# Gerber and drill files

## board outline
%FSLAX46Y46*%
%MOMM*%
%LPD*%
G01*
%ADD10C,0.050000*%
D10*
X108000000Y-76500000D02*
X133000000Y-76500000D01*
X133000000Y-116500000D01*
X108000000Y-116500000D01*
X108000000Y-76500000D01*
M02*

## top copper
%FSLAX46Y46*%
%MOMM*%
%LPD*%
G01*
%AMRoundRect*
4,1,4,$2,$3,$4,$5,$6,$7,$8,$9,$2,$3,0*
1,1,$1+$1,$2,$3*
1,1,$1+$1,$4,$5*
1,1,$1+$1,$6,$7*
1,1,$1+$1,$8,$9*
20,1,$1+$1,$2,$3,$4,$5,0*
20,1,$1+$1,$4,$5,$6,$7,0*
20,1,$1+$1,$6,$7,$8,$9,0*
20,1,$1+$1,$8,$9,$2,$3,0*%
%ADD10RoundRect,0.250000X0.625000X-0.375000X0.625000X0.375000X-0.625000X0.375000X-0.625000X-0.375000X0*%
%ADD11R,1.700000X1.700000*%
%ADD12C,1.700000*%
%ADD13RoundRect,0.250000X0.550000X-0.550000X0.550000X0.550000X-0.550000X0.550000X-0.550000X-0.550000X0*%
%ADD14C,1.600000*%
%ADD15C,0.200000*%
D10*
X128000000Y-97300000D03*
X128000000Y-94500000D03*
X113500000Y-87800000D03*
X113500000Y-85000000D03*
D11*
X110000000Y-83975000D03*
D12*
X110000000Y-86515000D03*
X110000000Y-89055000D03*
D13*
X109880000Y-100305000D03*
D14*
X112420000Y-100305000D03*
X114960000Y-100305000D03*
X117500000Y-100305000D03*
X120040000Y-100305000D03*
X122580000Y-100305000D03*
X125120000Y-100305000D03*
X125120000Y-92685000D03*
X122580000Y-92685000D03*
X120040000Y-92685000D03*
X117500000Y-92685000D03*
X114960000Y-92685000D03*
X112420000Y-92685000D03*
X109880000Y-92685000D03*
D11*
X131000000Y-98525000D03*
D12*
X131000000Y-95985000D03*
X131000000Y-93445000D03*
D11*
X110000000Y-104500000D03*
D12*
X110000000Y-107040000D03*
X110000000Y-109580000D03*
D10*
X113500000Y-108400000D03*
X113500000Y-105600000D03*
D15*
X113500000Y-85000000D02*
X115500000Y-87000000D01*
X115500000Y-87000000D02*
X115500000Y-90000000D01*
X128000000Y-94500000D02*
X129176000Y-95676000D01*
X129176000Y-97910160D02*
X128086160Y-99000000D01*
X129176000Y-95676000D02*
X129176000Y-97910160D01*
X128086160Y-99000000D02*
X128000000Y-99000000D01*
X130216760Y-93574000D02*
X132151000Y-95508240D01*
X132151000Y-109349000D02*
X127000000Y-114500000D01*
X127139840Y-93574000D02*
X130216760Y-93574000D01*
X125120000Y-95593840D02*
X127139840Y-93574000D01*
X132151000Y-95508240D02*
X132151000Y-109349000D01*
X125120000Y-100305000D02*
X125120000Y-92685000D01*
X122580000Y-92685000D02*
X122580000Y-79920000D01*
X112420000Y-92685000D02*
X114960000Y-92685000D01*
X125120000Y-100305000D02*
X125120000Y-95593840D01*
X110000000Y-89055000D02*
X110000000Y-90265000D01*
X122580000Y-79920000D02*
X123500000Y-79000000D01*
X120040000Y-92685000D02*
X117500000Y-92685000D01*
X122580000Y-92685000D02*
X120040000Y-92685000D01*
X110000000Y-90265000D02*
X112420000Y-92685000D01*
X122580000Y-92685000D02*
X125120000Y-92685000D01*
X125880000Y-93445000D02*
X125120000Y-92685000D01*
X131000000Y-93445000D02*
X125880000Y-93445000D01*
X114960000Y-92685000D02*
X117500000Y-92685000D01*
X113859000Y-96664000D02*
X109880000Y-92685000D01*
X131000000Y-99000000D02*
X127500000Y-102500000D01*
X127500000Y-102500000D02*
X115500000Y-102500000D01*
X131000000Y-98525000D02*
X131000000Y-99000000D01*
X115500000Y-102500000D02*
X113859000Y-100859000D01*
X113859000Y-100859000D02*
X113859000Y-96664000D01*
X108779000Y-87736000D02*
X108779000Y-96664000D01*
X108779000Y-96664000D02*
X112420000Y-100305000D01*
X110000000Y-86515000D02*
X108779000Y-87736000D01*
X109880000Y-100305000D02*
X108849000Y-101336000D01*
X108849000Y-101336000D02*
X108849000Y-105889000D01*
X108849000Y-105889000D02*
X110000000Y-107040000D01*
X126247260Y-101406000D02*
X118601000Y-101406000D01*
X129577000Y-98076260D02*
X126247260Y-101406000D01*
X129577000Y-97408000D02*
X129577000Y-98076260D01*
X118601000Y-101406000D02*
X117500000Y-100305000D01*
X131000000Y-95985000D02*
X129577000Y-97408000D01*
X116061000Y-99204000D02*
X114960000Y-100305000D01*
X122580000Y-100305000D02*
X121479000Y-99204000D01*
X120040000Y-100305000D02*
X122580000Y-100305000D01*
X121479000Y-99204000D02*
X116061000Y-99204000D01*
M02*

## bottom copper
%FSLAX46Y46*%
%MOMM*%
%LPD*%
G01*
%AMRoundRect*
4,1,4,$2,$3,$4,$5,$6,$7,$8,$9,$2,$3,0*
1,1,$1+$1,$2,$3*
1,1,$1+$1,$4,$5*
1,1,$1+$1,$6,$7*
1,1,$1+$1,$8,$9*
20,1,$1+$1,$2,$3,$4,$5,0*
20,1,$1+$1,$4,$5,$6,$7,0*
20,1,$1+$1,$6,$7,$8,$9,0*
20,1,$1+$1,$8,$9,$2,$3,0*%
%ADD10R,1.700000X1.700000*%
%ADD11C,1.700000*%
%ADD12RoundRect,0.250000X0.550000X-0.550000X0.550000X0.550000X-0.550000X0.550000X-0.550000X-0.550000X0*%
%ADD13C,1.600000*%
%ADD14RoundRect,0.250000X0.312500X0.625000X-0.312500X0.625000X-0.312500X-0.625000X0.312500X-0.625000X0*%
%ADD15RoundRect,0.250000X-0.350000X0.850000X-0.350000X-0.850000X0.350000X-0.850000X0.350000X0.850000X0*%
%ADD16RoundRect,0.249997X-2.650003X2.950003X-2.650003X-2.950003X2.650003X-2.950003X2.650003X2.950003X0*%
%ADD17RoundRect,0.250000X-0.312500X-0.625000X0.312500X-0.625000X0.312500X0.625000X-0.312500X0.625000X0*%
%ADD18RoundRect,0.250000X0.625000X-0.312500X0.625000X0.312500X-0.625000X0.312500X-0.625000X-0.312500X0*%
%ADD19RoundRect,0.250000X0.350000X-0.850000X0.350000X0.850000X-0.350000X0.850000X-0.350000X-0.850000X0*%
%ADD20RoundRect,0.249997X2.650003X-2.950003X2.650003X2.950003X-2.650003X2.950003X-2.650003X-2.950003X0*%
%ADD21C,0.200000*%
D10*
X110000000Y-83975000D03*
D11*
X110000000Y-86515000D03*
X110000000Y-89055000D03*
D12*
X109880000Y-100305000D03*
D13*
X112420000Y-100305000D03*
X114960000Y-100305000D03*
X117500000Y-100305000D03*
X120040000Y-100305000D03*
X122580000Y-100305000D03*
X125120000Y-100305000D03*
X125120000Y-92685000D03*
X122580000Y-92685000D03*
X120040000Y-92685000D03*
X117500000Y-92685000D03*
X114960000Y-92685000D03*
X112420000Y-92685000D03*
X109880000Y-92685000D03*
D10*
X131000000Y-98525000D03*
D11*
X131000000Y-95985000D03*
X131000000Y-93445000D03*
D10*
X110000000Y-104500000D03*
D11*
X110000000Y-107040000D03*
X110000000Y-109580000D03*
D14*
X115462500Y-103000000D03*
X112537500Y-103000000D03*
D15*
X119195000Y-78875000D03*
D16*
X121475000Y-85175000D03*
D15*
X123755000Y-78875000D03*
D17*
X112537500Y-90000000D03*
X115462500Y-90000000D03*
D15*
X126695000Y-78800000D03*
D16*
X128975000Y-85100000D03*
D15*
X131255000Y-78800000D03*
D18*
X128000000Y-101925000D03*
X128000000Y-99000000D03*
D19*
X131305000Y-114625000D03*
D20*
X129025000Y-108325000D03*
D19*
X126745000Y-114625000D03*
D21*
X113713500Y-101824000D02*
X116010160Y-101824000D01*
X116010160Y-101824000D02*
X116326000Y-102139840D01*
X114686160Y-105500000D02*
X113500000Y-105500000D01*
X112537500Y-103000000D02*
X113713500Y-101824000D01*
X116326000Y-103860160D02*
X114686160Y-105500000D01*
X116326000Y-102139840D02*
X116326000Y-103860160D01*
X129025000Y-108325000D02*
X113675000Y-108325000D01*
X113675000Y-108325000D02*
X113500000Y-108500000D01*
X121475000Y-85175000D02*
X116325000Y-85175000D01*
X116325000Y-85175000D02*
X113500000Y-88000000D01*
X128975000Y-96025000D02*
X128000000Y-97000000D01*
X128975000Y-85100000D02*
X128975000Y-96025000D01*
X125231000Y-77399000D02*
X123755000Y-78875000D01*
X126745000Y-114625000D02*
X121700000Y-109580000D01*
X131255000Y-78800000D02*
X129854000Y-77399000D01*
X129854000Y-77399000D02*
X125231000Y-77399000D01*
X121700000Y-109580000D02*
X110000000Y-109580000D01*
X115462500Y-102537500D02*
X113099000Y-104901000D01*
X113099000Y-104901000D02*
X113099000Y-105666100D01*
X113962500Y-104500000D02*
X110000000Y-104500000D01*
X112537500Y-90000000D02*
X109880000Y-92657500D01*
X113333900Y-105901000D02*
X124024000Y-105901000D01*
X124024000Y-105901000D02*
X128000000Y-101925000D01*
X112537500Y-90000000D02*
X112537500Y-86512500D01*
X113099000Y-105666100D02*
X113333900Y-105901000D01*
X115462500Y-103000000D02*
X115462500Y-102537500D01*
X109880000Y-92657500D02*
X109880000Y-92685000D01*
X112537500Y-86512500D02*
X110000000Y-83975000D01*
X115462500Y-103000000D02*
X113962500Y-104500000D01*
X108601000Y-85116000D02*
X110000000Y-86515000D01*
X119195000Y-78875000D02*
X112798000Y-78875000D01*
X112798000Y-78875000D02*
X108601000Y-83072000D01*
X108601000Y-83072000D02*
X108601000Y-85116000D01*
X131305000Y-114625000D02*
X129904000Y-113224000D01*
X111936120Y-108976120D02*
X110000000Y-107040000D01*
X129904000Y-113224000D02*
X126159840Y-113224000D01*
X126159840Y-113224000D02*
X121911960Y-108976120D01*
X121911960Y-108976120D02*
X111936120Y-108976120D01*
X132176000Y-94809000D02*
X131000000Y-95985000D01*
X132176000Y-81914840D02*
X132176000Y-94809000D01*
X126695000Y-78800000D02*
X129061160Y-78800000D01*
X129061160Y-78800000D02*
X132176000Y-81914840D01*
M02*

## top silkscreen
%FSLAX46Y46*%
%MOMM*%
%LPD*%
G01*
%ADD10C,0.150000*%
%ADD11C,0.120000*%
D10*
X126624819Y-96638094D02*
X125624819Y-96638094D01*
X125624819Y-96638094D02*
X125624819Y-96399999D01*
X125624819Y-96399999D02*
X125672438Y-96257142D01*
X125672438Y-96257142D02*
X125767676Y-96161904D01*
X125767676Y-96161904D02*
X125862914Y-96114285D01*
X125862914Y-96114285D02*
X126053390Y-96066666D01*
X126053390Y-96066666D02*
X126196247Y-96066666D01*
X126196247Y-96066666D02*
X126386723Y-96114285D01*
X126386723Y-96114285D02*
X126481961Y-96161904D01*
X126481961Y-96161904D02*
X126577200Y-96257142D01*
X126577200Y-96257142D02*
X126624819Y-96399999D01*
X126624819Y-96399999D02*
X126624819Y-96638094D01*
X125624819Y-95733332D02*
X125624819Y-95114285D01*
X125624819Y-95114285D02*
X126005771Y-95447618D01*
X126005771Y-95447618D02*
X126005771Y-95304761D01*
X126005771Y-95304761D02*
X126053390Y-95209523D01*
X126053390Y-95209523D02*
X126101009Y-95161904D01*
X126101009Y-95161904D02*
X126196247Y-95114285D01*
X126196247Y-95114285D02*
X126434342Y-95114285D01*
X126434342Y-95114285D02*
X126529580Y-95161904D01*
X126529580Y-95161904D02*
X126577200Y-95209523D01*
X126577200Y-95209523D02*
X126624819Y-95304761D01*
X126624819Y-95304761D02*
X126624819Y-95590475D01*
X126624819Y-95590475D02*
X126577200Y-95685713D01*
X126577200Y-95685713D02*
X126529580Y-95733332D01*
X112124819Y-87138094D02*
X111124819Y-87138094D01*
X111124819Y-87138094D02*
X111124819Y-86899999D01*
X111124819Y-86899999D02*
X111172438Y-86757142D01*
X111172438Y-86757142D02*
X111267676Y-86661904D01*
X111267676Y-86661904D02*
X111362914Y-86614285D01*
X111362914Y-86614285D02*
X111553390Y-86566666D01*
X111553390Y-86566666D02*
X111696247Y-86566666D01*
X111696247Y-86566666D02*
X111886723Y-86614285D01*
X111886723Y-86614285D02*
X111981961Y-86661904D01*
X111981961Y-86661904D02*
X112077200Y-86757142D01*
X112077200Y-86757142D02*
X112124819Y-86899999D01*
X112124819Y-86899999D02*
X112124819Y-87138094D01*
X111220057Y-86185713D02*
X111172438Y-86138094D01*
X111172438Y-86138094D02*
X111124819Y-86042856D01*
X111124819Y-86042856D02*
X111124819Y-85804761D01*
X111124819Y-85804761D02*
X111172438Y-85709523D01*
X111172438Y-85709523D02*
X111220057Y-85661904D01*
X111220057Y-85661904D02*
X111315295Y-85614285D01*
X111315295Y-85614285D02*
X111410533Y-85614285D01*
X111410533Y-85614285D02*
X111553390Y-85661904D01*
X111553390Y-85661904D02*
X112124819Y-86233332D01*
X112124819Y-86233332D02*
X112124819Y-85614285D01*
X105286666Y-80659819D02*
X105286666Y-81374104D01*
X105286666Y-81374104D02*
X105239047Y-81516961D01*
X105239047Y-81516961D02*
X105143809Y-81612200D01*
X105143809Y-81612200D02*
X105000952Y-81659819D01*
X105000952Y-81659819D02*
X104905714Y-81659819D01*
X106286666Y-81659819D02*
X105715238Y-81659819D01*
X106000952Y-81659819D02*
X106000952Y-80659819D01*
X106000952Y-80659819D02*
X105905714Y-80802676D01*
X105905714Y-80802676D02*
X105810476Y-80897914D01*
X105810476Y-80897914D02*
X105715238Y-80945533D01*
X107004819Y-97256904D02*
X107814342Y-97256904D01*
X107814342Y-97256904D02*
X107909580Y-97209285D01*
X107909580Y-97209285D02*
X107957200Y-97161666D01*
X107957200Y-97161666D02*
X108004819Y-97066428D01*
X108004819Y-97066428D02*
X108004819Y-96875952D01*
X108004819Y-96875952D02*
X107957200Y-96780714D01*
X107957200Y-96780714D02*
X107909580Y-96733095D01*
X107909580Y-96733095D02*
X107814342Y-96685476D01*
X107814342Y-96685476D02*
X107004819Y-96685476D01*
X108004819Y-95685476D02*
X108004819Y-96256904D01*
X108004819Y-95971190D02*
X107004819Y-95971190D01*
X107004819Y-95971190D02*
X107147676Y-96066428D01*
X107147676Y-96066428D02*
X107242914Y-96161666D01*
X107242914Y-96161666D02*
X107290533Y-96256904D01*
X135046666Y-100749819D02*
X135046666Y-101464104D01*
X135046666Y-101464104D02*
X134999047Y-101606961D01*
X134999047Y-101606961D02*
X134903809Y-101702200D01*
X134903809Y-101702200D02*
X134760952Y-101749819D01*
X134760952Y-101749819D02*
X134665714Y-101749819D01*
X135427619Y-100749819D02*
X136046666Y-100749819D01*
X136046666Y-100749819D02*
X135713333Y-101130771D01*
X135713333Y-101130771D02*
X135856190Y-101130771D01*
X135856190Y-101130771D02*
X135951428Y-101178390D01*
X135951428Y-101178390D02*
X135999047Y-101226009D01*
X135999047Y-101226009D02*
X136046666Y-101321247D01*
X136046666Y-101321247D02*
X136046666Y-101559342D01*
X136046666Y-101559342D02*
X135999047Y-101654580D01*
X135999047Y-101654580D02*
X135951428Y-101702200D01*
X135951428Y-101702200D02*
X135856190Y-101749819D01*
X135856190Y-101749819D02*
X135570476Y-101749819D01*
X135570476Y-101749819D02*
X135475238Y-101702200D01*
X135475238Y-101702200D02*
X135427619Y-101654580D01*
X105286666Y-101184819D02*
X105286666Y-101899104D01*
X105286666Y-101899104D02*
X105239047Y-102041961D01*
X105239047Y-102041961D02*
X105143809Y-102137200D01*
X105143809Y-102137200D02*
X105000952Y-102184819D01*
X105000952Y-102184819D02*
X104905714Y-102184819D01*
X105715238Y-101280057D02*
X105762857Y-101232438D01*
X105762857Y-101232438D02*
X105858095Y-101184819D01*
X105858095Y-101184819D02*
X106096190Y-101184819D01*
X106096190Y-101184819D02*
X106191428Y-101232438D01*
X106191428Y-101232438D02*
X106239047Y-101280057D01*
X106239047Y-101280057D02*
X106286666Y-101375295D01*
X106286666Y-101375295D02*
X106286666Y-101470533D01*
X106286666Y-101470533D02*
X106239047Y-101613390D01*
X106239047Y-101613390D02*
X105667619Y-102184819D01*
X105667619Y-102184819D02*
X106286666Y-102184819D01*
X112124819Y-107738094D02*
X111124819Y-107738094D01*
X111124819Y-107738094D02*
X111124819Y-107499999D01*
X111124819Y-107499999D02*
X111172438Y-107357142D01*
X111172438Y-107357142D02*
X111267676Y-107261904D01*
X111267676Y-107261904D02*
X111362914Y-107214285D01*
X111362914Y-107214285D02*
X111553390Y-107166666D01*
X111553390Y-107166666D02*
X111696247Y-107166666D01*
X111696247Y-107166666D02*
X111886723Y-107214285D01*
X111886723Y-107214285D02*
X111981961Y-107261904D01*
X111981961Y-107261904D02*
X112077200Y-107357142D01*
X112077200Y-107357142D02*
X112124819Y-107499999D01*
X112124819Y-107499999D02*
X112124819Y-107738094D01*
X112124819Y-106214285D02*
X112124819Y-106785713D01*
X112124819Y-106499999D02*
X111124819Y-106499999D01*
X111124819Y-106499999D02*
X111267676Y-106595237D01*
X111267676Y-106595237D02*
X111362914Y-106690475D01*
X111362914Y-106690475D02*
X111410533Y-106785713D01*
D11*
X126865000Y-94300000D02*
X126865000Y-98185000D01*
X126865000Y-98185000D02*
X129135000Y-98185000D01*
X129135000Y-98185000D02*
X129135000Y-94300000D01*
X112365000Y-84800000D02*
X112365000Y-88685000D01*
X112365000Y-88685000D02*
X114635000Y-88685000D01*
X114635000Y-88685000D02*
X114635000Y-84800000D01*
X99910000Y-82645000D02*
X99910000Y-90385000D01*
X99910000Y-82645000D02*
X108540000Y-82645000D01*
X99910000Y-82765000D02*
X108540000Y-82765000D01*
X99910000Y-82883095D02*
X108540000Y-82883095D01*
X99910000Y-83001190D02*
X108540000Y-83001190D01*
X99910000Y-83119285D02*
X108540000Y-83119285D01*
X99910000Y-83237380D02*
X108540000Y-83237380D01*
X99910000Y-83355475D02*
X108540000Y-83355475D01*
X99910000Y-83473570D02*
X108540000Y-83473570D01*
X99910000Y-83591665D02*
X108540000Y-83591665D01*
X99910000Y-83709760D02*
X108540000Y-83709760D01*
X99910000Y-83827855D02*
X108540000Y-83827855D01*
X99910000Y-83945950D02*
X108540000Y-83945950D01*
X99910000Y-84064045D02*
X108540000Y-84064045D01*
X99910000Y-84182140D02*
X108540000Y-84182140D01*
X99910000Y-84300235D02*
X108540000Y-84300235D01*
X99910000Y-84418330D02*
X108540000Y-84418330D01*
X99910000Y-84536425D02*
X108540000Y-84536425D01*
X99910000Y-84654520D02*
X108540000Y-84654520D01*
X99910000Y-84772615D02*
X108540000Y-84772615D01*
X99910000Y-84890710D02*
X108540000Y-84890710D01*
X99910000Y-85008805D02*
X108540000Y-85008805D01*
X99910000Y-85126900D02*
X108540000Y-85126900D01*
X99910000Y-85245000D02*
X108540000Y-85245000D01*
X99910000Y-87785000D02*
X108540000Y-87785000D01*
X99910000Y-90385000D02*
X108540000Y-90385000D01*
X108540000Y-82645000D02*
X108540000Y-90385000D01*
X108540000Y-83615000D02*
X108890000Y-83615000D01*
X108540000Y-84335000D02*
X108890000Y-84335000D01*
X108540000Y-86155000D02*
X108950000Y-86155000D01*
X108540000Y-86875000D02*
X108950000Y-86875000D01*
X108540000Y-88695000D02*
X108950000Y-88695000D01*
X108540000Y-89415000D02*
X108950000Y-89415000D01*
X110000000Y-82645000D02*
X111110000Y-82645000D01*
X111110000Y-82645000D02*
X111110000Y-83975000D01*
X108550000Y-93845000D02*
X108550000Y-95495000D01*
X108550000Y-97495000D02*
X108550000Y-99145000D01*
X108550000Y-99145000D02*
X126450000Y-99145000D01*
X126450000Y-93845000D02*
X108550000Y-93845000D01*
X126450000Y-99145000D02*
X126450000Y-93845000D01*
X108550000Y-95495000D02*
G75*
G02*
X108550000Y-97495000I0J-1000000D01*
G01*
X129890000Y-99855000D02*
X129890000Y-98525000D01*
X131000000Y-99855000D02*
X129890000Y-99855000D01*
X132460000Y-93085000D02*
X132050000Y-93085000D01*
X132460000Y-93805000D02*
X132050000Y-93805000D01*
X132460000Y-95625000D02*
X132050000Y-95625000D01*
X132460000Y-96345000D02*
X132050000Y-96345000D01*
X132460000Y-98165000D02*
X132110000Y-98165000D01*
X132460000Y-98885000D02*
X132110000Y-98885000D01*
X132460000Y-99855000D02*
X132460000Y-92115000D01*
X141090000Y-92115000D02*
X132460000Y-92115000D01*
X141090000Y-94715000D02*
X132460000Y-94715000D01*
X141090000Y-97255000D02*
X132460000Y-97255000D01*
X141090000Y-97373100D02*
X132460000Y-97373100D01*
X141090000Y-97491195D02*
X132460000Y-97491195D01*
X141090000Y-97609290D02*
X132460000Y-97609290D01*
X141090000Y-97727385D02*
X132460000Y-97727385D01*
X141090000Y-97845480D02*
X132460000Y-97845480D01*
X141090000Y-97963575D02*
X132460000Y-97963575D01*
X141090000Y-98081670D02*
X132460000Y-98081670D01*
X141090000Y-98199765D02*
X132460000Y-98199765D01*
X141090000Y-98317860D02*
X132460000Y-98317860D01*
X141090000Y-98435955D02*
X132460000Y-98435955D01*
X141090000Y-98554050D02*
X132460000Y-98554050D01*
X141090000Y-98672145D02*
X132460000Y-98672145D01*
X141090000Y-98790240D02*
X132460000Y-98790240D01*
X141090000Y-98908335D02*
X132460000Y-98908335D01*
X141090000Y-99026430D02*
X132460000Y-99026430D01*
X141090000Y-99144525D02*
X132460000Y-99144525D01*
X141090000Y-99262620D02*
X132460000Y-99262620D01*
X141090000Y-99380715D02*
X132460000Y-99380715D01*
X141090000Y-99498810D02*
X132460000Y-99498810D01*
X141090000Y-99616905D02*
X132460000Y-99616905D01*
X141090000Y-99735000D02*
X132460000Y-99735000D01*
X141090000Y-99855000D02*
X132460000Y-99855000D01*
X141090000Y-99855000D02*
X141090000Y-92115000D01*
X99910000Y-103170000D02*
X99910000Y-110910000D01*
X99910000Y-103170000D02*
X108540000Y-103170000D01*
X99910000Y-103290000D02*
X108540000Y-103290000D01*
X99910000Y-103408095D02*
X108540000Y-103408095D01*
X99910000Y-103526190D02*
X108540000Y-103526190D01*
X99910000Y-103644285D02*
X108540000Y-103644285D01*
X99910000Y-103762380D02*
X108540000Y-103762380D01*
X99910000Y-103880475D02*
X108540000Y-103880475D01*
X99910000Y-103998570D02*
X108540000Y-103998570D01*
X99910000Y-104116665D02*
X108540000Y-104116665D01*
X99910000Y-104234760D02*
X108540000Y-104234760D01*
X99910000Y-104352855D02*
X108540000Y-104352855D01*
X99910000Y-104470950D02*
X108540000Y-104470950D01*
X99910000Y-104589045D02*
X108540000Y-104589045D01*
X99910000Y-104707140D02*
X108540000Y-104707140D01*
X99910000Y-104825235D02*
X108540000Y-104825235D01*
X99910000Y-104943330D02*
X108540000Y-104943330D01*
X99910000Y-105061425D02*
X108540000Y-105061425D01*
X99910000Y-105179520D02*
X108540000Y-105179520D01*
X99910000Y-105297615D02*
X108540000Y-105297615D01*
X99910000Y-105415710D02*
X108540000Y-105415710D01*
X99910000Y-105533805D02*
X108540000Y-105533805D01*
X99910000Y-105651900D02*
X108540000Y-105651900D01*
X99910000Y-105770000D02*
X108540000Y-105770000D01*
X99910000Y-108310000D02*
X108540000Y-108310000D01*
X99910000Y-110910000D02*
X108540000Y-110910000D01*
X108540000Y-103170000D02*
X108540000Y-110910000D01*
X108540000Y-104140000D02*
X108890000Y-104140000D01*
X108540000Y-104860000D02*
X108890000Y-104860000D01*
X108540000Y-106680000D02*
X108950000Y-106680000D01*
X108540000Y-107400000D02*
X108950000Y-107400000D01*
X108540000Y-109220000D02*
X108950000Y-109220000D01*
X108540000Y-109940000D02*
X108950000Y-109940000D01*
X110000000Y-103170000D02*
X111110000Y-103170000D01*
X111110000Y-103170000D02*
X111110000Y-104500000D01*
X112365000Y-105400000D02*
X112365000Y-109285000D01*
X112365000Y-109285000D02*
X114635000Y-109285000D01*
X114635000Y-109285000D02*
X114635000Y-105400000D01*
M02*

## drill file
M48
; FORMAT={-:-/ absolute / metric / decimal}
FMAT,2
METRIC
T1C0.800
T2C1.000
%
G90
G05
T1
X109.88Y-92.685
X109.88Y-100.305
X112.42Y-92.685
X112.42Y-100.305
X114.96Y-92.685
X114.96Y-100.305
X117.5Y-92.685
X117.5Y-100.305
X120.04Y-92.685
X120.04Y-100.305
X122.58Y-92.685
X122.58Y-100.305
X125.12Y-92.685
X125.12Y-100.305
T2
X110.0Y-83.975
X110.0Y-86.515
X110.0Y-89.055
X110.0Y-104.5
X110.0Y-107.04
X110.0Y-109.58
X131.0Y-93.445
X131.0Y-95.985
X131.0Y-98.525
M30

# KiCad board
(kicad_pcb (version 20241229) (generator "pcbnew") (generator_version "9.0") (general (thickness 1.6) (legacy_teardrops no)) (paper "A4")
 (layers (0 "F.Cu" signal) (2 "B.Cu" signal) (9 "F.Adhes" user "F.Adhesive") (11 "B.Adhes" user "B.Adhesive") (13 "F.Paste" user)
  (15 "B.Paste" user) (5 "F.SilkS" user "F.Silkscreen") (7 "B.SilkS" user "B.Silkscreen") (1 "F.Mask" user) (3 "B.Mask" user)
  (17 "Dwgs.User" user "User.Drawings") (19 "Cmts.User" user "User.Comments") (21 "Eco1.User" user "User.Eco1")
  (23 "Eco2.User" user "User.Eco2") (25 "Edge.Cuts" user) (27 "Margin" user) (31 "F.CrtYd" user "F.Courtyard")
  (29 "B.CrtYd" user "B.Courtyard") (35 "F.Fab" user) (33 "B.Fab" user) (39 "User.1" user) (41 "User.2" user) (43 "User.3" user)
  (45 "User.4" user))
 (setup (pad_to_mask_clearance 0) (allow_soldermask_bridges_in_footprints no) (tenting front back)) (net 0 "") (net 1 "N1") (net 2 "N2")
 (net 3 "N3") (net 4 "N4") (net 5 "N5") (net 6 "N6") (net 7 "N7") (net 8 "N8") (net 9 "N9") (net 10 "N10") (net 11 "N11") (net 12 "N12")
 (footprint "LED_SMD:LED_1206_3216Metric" (layer "F.Cu") (at 128 95.9 90)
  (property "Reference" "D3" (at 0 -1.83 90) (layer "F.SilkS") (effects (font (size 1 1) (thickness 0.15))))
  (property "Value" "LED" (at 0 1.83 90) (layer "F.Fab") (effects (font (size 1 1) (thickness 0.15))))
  (fp_line (start 1.6 -1.135) (end -2.285 -1.135) (stroke (width 0.12) (type solid)) (layer "F.SilkS"))
  (fp_line (start -2.285 -1.135) (end -2.285 1.135) (stroke (width 0.12) (type solid)) (layer "F.SilkS"))
  (fp_line (start -2.285 1.135) (end 1.6 1.135) (stroke (width 0.12) (type solid)) (layer "F.SilkS"))
  (pad "1" smd roundrect (at -1.4 0 90) (size 1.25 1.75) (layers "F.Cu" "F.Mask" "F.Paste") (roundrect_rratio 0.2) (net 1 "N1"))
  (pad "2" smd roundrect (at 1.4 0 90) (size 1.25 1.75) (layers "F.Cu" "F.Mask" "F.Paste") (roundrect_rratio 0.2) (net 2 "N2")))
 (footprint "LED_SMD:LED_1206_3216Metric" (layer "F.Cu") (at 113.5 86.4 90)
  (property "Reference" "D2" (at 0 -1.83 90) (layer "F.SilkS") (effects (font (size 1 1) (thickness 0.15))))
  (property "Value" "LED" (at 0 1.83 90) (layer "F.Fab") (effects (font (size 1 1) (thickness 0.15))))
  (fp_line (start 1.6 -1.135) (end -2.285 -1.135) (stroke (width 0.12) (type solid)) (layer "F.SilkS"))
  (fp_line (start -2.285 -1.135) (end -2.285 1.135) (stroke (width 0.12) (type solid)) (layer "F.SilkS"))
  (fp_line (start -2.285 1.135) (end 1.6 1.135) (stroke (width 0.12) (type solid)) (layer "F.SilkS"))
  (pad "1" smd roundrect (at -1.4 0 90) (size 1.25 1.75) (layers "F.Cu" "F.Mask" "F.Paste") (roundrect_rratio 0.2) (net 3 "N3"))
  (pad "2" smd roundrect (at 1.4 0 90) (size 1.25 1.75) (layers "F.Cu" "F.Mask" "F.Paste") (roundrect_rratio 0.2) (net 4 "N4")))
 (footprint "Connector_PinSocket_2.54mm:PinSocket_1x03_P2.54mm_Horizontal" (layer "F.Cu") (at 110 83.975)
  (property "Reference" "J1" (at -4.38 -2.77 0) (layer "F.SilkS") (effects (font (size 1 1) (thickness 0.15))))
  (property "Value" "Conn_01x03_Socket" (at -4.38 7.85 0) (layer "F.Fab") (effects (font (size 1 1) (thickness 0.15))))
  (fp_line (start -10.09 -1.33) (end -10.09 6.41) (stroke (width 0.12) (type solid)) (layer "F.SilkS"))
  (fp_line (start -10.09 -1.33) (end -1.46 -1.33) (stroke (width 0.12) (type solid)) (layer "F.SilkS"))
  (fp_line (start -10.09 -1.21) (end -1.46 -1.21) (stroke (width 0.12) (type solid)) (layer "F.SilkS"))
  (fp_line (start -10.09 -1.091905) (end -1.46 -1.091905) (stroke (width 0.12) (type solid)) (layer "F.SilkS"))
  (fp_line (start -10.09 -0.97381) (end -1.46 -0.97381) (stroke (width 0.12) (type solid)) (layer "F.SilkS"))
  (fp_line (start -10.09 -0.855715) (end -1.46 -0.855715) (stroke (width 0.12) (type solid)) (layer "F.SilkS"))
  (fp_line (start -10.09 -0.73762) (end -1.46 -0.73762) (stroke (width 0.12) (type solid)) (layer "F.SilkS"))
  (fp_line (start -10.09 -0.619525) (end -1.46 -0.619525) (stroke (width 0.12) (type solid)) (layer "F.SilkS"))
  (fp_line (start -10.09 -0.50143) (end -1.46 -0.50143) (stroke (width 0.12) (type solid)) (layer "F.SilkS"))
  (fp_line (start -10.09 -0.383335) (end -1.46 -0.383335) (stroke (width 0.12) (type solid)) (layer "F.SilkS"))
  (fp_line (start -10.09 -0.26524) (end -1.46 -0.26524) (stroke (width 0.12) (type solid)) (layer "F.SilkS"))
  (fp_line (start -10.09 -0.147145) (end -1.46 -0.147145) (stroke (width 0.12) (type solid)) (layer "F.SilkS"))
  (fp_line (start -10.09 -0.02905) (end -1.46 -0.02905) (stroke (width 0.12) (type solid)) (layer "F.SilkS"))
  (fp_line (start -10.09 0.089045) (end -1.46 0.089045) (stroke (width 0.12) (type solid)) (layer "F.SilkS"))
  (fp_line (start -10.09 0.20714) (end -1.46 0.20714) (stroke (width 0.12) (type solid)) (layer "F.SilkS"))
  (fp_line (start -10.09 0.325235) (end -1.46 0.325235) (stroke (width 0.12) (type solid)) (layer "F.SilkS"))
  (fp_line (start -10.09 0.44333) (end -1.46 0.44333) (stroke (width 0.12) (type solid)) (layer "F.SilkS"))
  (fp_line (start -10.09 0.561425) (end -1.46 0.561425) (stroke (width 0.12) (type solid)) (layer "F.SilkS"))
  (fp_line (start -10.09 0.67952) (end -1.46 0.67952) (stroke (width 0.12) (type solid)) (layer "F.SilkS"))
  (fp_line (start -10.09 0.797615) (end -1.46 0.797615) (stroke (width 0.12) (type solid)) (layer "F.SilkS"))
  (fp_line (start -10.09 0.91571) (end -1.46 0.91571) (stroke (width 0.12) (type solid)) (layer "F.SilkS"))
  (fp_line (start -10.09 1.033805) (end -1.46 1.033805) (stroke (width 0.12) (type solid)) (layer "F.SilkS"))
  (fp_line (start -10.09 1.1519) (end -1.46 1.1519) (stroke (width 0.12) (type solid)) (layer "F.SilkS"))
  (fp_line (start -10.09 1.27) (end -1.46 1.27) (stroke (width 0.12) (type solid)) (layer "F.SilkS"))
  (fp_line (start -10.09 3.81) (end -1.46 3.81) (stroke (width 0.12) (type solid)) (layer "F.SilkS"))
  (fp_line (start -10.09 6.41) (end -1.46 6.41) (stroke (width 0.12) (type solid)) (layer "F.SilkS"))
  (fp_line (start -1.46 -1.33) (end -1.46 6.41) (stroke (width 0.12) (type solid)) (layer "F.SilkS"))
  (fp_line (start -1.46 -0.36) (end -1.11 -0.36) (stroke (width 0.12) (type solid)) (layer "F.SilkS"))
  (fp_line (start -1.46 0.36) (end -1.11 0.36) (stroke (width 0.12) (type solid)) (layer "F.SilkS"))
  (fp_line (start -1.46 2.18) (end -1.05 2.18) (stroke (width 0.12) (type solid)) (layer "F.SilkS"))
  (fp_line (start -1.46 2.9) (end -1.05 2.9) (stroke (width 0.12) (type solid)) (layer "F.SilkS"))
  (fp_line (start -1.46 4.72) (end -1.05 4.72) (stroke (width 0.12) (type solid)) (layer "F.SilkS"))
  (fp_line (start -1.46 5.44) (end -1.05 5.44) (stroke (width 0.12) (type solid)) (layer "F.SilkS"))
  (fp_line (start 0 -1.33) (end 1.11 -1.33) (stroke (width 0.12) (type solid)) (layer "F.SilkS"))
  (fp_line (start 1.11 -1.33) (end 1.11 0) (stroke (width 0.12) (type solid)) (layer "F.SilkS"))
  (pad "1" thru_hole rect (at 0 0) (size 1.7 1.7) (drill 1) (layers "*.Cu" "*.Mask") (remove_unused_layers no) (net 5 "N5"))
  (pad "2" thru_hole circle (at 0 2.54) (size 1.7 1.7) (drill 1) (layers "*.Cu" "*.Mask") (remove_unused_layers no) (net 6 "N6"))
  (pad "3" thru_hole circle (at 0 5.08) (size 1.7 1.7) (drill 1) (layers "*.Cu" "*.Mask") (remove_unused_layers no) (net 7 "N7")))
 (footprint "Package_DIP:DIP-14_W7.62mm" (layer "F.Cu") (at 109.88 100.305 90)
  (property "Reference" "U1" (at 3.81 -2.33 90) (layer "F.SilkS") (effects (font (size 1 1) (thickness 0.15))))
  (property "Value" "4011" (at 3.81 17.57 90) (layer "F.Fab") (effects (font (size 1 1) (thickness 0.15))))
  (fp_line (start 6.46 -1.33) (end 4.81 -1.33) (stroke (width 0.12) (type solid)) (layer "F.SilkS"))
  (fp_line (start 2.81 -1.33) (end 1.16 -1.33) (stroke (width 0.12) (type solid)) (layer "F.SilkS"))
  (fp_line (start 1.16 -1.33) (end 1.16 16.57) (stroke (width 0.12) (type solid)) (layer "F.SilkS"))
  (fp_line (start 6.46 16.57) (end 6.46 -1.33) (stroke (width 0.12) (type solid)) (layer "F.SilkS"))
  (fp_line (start 1.16 16.57) (end 6.46 16.57) (stroke (width 0.12) (type solid)) (layer "F.SilkS"))
  (fp_arc (start 4.81 -1.33) (mid 3.81 -0.33) (end 2.81 -1.33) (stroke (width 0.12) (type solid)) (layer "F.SilkS"))
  (pad "1" thru_hole roundrect (at 0 0 90) (size 1.6 1.6) (drill 0.8) (layers "*.Cu" "*.Mask") (remove_unused_layers no)
   (roundrect_rratio 0.15625) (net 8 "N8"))
  (pad "2" thru_hole circle (at 0 2.54 90) (size 1.6 1.6) (drill 0.8) (layers "*.Cu" "*.Mask") (remove_unused_layers no) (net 6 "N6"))
  (pad "3" thru_hole circle (at 0 5.08 90) (size 1.6 1.6) (drill 0.8) (layers "*.Cu" "*.Mask") (remove_unused_layers no) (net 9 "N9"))
  (pad "4" thru_hole circle (at 0 7.62 90) (size 1.6 1.6) (drill 0.8) (layers "*.Cu" "*.Mask") (remove_unused_layers no) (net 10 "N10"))
  (pad "5" thru_hole circle (at 0 10.16 90) (size 1.6 1.6) (drill 0.8) (layers "*.Cu" "*.Mask") (remove_unused_layers no) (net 9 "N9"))
  (pad "6" thru_hole circle (at 0 12.7 90) (size 1.6 1.6) (drill 0.8) (layers "*.Cu" "*.Mask") (remove_unused_layers no) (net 9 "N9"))
  (pad "7" thru_hole circle (at 0 15.24 90) (size 1.6 1.6) (drill 0.8) (layers "*.Cu" "*.Mask") (remove_unused_layers no) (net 7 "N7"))
  (pad "8" thru_hole circle (at 7.62 15.24 90) (size 1.6 1.6) (drill 0.8) (layers "*.Cu" "*.Mask") (remove_unused_layers no) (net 7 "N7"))
  (pad "9" thru_hole circle (at 7.62 12.7 90) (size 1.6 1.6) (drill 0.8) (layers "*.Cu" "*.Mask") (remove_unused_layers no) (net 7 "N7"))
  (pad "10" thru_hole circle (at 7.62 10.16 90) (size 1.6 1.6) (drill 0.8) (layers "*.Cu" "*.Mask") (remove_unused_layers no) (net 7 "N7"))
  (pad "11" thru_hole circle (at 7.62 7.62 90) (size 1.6 1.6) (drill 0.8) (layers "*.Cu" "*.Mask") (remove_unused_layers no) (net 7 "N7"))
  (pad "12" thru_hole circle (at 7.62 5.08 90) (size 1.6 1.6) (drill 0.8) (layers "*.Cu" "*.Mask") (remove_unused_layers no) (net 7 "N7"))
  (pad "13" thru_hole circle (at 7.62 2.54 90) (size 1.6 1.6) (drill 0.8) (layers "*.Cu" "*.Mask") (remove_unused_layers no) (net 7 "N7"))
  (pad "14" thru_hole circle (at 7.62 0 90) (size 1.6 1.6) (drill 0.8) (layers "*.Cu" "*.Mask") (remove_unused_layers no) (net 5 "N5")))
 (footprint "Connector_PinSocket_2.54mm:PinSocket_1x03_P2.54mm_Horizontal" (layer "F.Cu") (at 131 98.525 180)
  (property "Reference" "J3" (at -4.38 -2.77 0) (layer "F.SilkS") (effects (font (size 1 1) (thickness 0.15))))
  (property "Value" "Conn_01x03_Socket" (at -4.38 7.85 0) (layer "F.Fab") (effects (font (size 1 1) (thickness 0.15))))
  (fp_line (start 1.11 -1.33) (end 1.11 0) (stroke (width 0.12) (type solid)) (layer "F.SilkS"))
  (fp_line (start 0 -1.33) (end 1.11 -1.33) (stroke (width 0.12) (type solid)) (layer "F.SilkS"))
  (fp_line (start -1.46 5.44) (end -1.05 5.44) (stroke (width 0.12) (type solid)) (layer "F.SilkS"))
  (fp_line (start -1.46 4.72) (end -1.05 4.72) (stroke (width 0.12) (type solid)) (layer "F.SilkS"))
  (fp_line (start -1.46 2.9) (end -1.05 2.9) (stroke (width 0.12) (type solid)) (layer "F.SilkS"))
  (fp_line (start -1.46 2.18) (end -1.05 2.18) (stroke (width 0.12) (type solid)) (layer "F.SilkS"))
  (fp_line (start -1.46 0.36) (end -1.11 0.36) (stroke (width 0.12) (type solid)) (layer "F.SilkS"))
  (fp_line (start -1.46 -0.36) (end -1.11 -0.36) (stroke (width 0.12) (type solid)) (layer "F.SilkS"))
  (fp_line (start -1.46 -1.33) (end -1.46 6.41) (stroke (width 0.12) (type solid)) (layer "F.SilkS"))
  (fp_line (start -10.09 6.41) (end -1.46 6.41) (stroke (width 0.12) (type solid)) (layer "F.SilkS"))
  (fp_line (start -10.09 3.81) (end -1.46 3.81) (stroke (width 0.12) (type solid)) (layer "F.SilkS"))
  (fp_line (start -10.09 1.27) (end -1.46 1.27) (stroke (width 0.12) (type solid)) (layer "F.SilkS"))
  (fp_line (start -10.09 1.1519) (end -1.46 1.1519) (stroke (width 0.12) (type solid)) (layer "F.SilkS"))
  (fp_line (start -10.09 1.033805) (end -1.46 1.033805) (stroke (width 0.12) (type solid)) (layer "F.SilkS"))
  (fp_line (start -10.09 0.91571) (end -1.46 0.91571) (stroke (width 0.12) (type solid)) (layer "F.SilkS"))
  (fp_line (start -10.09 0.797615) (end -1.46 0.797615) (stroke (width 0.12) (type solid)) (layer "F.SilkS"))
  (fp_line (start -10.09 0.67952) (end -1.46 0.67952) (stroke (width 0.12) (type solid)) (layer "F.SilkS"))
  (fp_line (start -10.09 0.561425) (end -1.46 0.561425) (stroke (width 0.12) (type solid)) (layer "F.SilkS"))
  (fp_line (start -10.09 0.44333) (end -1.46 0.44333) (stroke (width 0.12) (type solid)) (layer "F.SilkS"))
  (fp_line (start -10.09 0.325235) (end -1.46 0.325235) (stroke (width 0.12) (type solid)) (layer "F.SilkS"))
  (fp_line (start -10.09 0.20714) (end -1.46 0.20714) (stroke (width 0.12) (type solid)) (layer "F.SilkS"))
  (fp_line (start -10.09 0.089045) (end -1.46 0.089045) (stroke (width 0.12) (type solid)) (layer "F.SilkS"))
  (fp_line (start -10.09 -0.02905) (end -1.46 -0.02905) (stroke (width 0.12) (type solid)) (layer "F.SilkS"))
  (fp_line (start -10.09 -0.147145) (end -1.46 -0.147145) (stroke (width 0.12) (type solid)) (layer "F.SilkS"))
  (fp_line (start -10.09 -0.26524) (end -1.46 -0.26524) (stroke (width 0.12) (type solid)) (layer "F.SilkS"))
  (fp_line (start -10.09 -0.383335) (end -1.46 -0.383335) (stroke (width 0.12) (type solid)) (layer "F.SilkS"))
  (fp_line (start -10.09 -0.50143) (end -1.46 -0.50143) (stroke (width 0.12) (type solid)) (layer "F.SilkS"))
  (fp_line (start -10.09 -0.619525) (end -1.46 -0.619525) (stroke (width 0.12) (type solid)) (layer "F.SilkS"))
  (fp_line (start -10.09 -0.73762) (end -1.46 -0.73762) (stroke (width 0.12) (type solid)) (layer "F.SilkS"))
  (fp_line (start -10.09 -0.855715) (end -1.46 -0.855715) (stroke (width 0.12) (type solid)) (layer "F.SilkS"))
  (fp_line (start -10.09 -0.97381) (end -1.46 -0.97381) (stroke (width 0.12) (type solid)) (layer "F.SilkS"))
  (fp_line (start -10.09 -1.091905) (end -1.46 -1.091905) (stroke (width 0.12) (type solid)) (layer "F.SilkS"))
  (fp_line (start -10.09 -1.21) (end -1.46 -1.21) (stroke (width 0.12) (type solid)) (layer "F.SilkS"))
  (fp_line (start -10.09 -1.33) (end -1.46 -1.33) (stroke (width 0.12) (type solid)) (layer "F.SilkS"))
  (fp_line (start -10.09 -1.33) (end -10.09 6.41) (stroke (width 0.12) (type solid)) (layer "F.SilkS"))
  (pad "1" thru_hole rect (at 0 0 180) (size 1.7 1.7) (drill 1) (layers "*.Cu" "*.Mask") (remove_unused_layers no) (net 5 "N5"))
  (pad "2" thru_hole circle (at 0 2.54 180) (size 1.7 1.7) (drill 1) (layers "*.Cu" "*.Mask") (remove_unused_layers no) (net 10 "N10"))
  (pad "3" thru_hole circle (at 0 5.08 180) (size 1.7 1.7) (drill 1) (layers "*.Cu" "*.Mask") (remove_unused_layers no) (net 7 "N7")))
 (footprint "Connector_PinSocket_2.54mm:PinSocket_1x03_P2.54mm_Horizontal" (layer "F.Cu") (at 110 104.5)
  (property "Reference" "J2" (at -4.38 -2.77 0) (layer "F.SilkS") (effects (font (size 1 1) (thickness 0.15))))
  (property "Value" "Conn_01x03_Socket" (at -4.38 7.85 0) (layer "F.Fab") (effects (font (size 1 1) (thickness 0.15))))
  (fp_line (start -10.09 -1.33) (end -10.09 6.41) (stroke (width 0.12) (type solid)) (layer "F.SilkS"))
  (fp_line (start -10.09 -1.33) (end -1.46 -1.33) (stroke (width 0.12) (type solid)) (layer "F.SilkS"))
  (fp_line (start -10.09 -1.21) (end -1.46 -1.21) (stroke (width 0.12) (type solid)) (layer "F.SilkS"))
  (fp_line (start -10.09 -1.091905) (end -1.46 -1.091905) (stroke (width 0.12) (type solid)) (layer "F.SilkS"))
  (fp_line (start -10.09 -0.97381) (end -1.46 -0.97381) (stroke (width 0.12) (type solid)) (layer "F.SilkS"))
  (fp_line (start -10.09 -0.855715) (end -1.46 -0.855715) (stroke (width 0.12) (type solid)) (layer "F.SilkS"))
  (fp_line (start -10.09 -0.73762) (end -1.46 -0.73762) (stroke (width 0.12) (type solid)) (layer "F.SilkS"))
  (fp_line (start -10.09 -0.619525) (end -1.46 -0.619525) (stroke (width 0.12) (type solid)) (layer "F.SilkS"))
  (fp_line (start -10.09 -0.50143) (end -1.46 -0.50143) (stroke (width 0.12) (type solid)) (layer "F.SilkS"))
  (fp_line (start -10.09 -0.383335) (end -1.46 -0.383335) (stroke (width 0.12) (type solid)) (layer "F.SilkS"))
  (fp_line (start -10.09 -0.26524) (end -1.46 -0.26524) (stroke (width 0.12) (type solid)) (layer "F.SilkS"))
  (fp_line (start -10.09 -0.147145) (end -1.46 -0.147145) (stroke (width 0.12) (type solid)) (layer "F.SilkS"))
  (fp_line (start -10.09 -0.02905) (end -1.46 -0.02905) (stroke (width 0.12) (type solid)) (layer "F.SilkS"))
  (fp_line (start -10.09 0.089045) (end -1.46 0.089045) (stroke (width 0.12) (type solid)) (layer "F.SilkS"))
  (fp_line (start -10.09 0.20714) (end -1.46 0.20714) (stroke (width 0.12) (type solid)) (layer "F.SilkS"))
  (fp_line (start -10.09 0.325235) (end -1.46 0.325235) (stroke (width 0.12) (type solid)) (layer "F.SilkS"))
  (fp_line (start -10.09 0.44333) (end -1.46 0.44333) (stroke (width 0.12) (type solid)) (layer "F.SilkS"))
  (fp_line (start -10.09 0.561425) (end -1.46 0.561425) (stroke (width 0.12) (type solid)) (layer "F.SilkS"))
  (fp_line (start -10.09 0.67952) (end -1.46 0.67952) (stroke (width 0.12) (type solid)) (layer "F.SilkS"))
  (fp_line (start -10.09 0.797615) (end -1.46 0.797615) (stroke (width 0.12) (type solid)) (layer "F.SilkS"))
  (fp_line (start -10.09 0.91571) (end -1.46 0.91571) (stroke (width 0.12) (type solid)) (layer "F.SilkS"))
  (fp_line (start -10.09 1.033805) (end -1.46 1.033805) (stroke (width 0.12) (type solid)) (layer "F.SilkS"))
  (fp_line (start -10.09 1.1519) (end -1.46 1.1519) (stroke (width 0.12) (type solid)) (layer "F.SilkS"))
  (fp_line (start -10.09 1.27) (end -1.46 1.27) (stroke (width 0.12) (type solid)) (layer "F.SilkS"))
  (fp_line (start -10.09 3.81) (end -1.46 3.81) (stroke (width 0.12) (type solid)) (layer "F.SilkS"))
  (fp_line (start -10.09 6.41) (end -1.46 6.41) (stroke (width 0.12) (type solid)) (layer "F.SilkS"))
  (fp_line (start -1.46 -1.33) (end -1.46 6.41) (stroke (width 0.12) (type solid)) (layer "F.SilkS"))
  (fp_line (start -1.46 -0.36) (end -1.11 -0.36) (stroke (width 0.12) (type solid)) (layer "F.SilkS"))
  (fp_line (start -1.46 0.36) (end -1.11 0.36) (stroke (width 0.12) (type solid)) (layer "F.SilkS"))
  (fp_line (start -1.46 2.18) (end -1.05 2.18) (stroke (width 0.12) (type solid)) (layer "F.SilkS"))
  (fp_line (start -1.46 2.9) (end -1.05 2.9) (stroke (width 0.12) (type solid)) (layer "F.SilkS"))
  (fp_line (start -1.46 4.72) (end -1.05 4.72) (stroke (width 0.12) (type solid)) (layer "F.SilkS"))
  (fp_line (start -1.46 5.44) (end -1.05 5.44) (stroke (width 0.12) (type solid)) (layer "F.SilkS"))
  (fp_line (start 0 -1.33) (end 1.11 -1.33) (stroke (width 0.12) (type solid)) (layer "F.SilkS"))
  (fp_line (start 1.11 -1.33) (end 1.11 0) (stroke (width 0.12) (type solid)) (layer "F.SilkS"))
  (pad "1" thru_hole rect (at 0 0) (size 1.7 1.7) (drill 1) (layers "*.Cu" "*.Mask") (remove_unused_layers no) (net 5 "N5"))
  (pad "2" thru_hole circle (at 0 2.54) (size 1.7 1.7) (drill 1) (layers "*.Cu" "*.Mask") (remove_unused_layers no) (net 8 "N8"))
  (pad "3" thru_hole circle (at 0 5.08) (size 1.7 1.7) (drill 1) (layers "*.Cu" "*.Mask") (remove_unused_layers no) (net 7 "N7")))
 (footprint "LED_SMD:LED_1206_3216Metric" (layer "F.Cu") (at 113.5 107 90)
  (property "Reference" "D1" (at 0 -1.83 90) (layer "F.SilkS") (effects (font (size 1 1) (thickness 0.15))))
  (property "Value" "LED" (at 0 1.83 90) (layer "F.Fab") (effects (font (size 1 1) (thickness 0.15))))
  (fp_line (start 1.6 -1.135) (end -2.285 -1.135) (stroke (width 0.12) (type solid)) (layer "F.SilkS"))
  (fp_line (start -2.285 -1.135) (end -2.285 1.135) (stroke (width 0.12) (type solid)) (layer "F.SilkS"))
  (fp_line (start -2.285 1.135) (end 1.6 1.135) (stroke (width 0.12) (type solid)) (layer "F.SilkS"))
  (pad "1" smd roundrect (at -1.4 0 90) (size 1.25 1.75) (layers "F.Cu" "F.Mask" "F.Paste") (roundrect_rratio 0.2) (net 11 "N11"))
  (pad "2" smd roundrect (at 1.4 0 90) (size 1.25 1.75) (layers "F.Cu" "F.Mask" "F.Paste") (roundrect_rratio 0.2) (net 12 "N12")))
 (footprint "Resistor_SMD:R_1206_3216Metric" (layer "B.Cu") (at 114 103 180)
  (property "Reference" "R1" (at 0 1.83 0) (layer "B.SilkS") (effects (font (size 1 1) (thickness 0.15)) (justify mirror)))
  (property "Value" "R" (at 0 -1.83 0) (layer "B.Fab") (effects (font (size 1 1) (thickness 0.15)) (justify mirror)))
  (pad "1" smd roundrect (at -1.4625 0 180) (size 1.125 1.75) (layers "B.Cu" "B.Mask" "B.Paste") (roundrect_rratio 0.222222) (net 5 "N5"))
  (pad "2" smd roundrect (at 1.4625 0 180) (size 1.125 1.75) (layers "B.Cu" "B.Mask" "B.Paste") (roundrect_rratio 0.222222) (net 12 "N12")))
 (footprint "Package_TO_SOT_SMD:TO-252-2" (layer "B.Cu") (at 121.475 83.915 -90)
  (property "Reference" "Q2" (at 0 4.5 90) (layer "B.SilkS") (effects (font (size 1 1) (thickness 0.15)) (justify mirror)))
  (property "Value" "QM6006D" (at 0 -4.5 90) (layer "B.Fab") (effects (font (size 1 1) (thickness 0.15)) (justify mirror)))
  (pad "" smd roundrect (at -0.415 -1.525 270) (size 3.05 2.75) (layers "B.Paste") (roundrect_rratio 0.090909))
  (pad "" smd roundrect (at -0.415 1.525 270) (size 3.05 2.75) (layers "B.Paste") (roundrect_rratio 0.090909))
  (pad "" smd roundrect (at 2.935 -1.525 270) (size 3.05 2.75) (layers "B.Paste") (roundrect_rratio 0.090909))
  (pad "" smd roundrect (at 2.935 1.525 270) (size 3.05 2.75) (layers "B.Paste") (roundrect_rratio 0.090909))
  (pad "1" smd roundrect (at -5.04 2.28 270) (size 2.2 1.2) (layers "B.Cu" "B.Mask" "B.Paste") (roundrect_rratio 0.208333) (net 6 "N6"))
  (pad "2" smd roundrect (at 1.26 0 270) (size 6.4 5.8) (layers "B.Cu" "B.Mask") (roundrect_rratio 0.043103) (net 3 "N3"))
  (pad "3" smd roundrect (at -5.04 -2.28 270) (size 2.2 1.2) (layers "B.Cu" "B.Mask" "B.Paste") (roundrect_rratio 0.208333) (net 7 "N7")))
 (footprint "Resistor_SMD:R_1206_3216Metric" (layer "B.Cu") (at 114 90)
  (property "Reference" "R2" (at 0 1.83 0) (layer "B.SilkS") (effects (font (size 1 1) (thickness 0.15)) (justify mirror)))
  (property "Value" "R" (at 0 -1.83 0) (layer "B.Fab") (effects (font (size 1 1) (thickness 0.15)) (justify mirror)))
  (pad "1" smd roundrect (at -1.4625 0) (size 1.125 1.75) (layers "B.Cu" "B.Mask" "B.Paste") (roundrect_rratio 0.222222) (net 5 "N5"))
  (pad "2" smd roundrect (at 1.4625 0) (size 1.125 1.75) (layers "B.Cu" "B.Mask" "B.Paste") (roundrect_rratio 0.222222) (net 4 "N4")))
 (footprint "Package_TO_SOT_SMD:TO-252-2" (layer "B.Cu") (at 128.975 83.84 -90)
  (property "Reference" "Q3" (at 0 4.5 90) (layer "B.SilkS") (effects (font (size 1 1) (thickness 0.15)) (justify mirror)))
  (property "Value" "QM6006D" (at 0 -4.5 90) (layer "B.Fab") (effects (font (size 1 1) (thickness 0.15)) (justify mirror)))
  (pad "" smd roundrect (at -0.415 -1.525 270) (size 3.05 2.75) (layers "B.Paste") (roundrect_rratio 0.090909))
  (pad "" smd roundrect (at -0.415 1.525 270) (size 3.05 2.75) (layers "B.Paste") (roundrect_rratio 0.090909))
  (pad "" smd roundrect (at 2.935 -1.525 270) (size 3.05 2.75) (layers "B.Paste") (roundrect_rratio 0.090909))
  (pad "" smd roundrect (at 2.935 1.525 270) (size 3.05 2.75) (layers "B.Paste") (roundrect_rratio 0.090909))
  (pad "1" smd roundrect (at -5.04 2.28 270) (size 2.2 1.2) (layers "B.Cu" "B.Mask" "B.Paste") (roundrect_rratio 0.208333) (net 10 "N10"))
  (pad "2" smd roundrect (at 1.26 0 270) (size 6.4 5.8) (layers "B.Cu" "B.Mask") (roundrect_rratio 0.043103) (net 1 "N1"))
  (pad "3" smd roundrect (at -5.04 -2.28 270) (size 2.2 1.2) (layers "B.Cu" "B.Mask" "B.Paste") (roundrect_rratio 0.208333) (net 7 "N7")))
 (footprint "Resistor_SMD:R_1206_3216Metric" (layer "B.Cu") (at 128 100.4625 90)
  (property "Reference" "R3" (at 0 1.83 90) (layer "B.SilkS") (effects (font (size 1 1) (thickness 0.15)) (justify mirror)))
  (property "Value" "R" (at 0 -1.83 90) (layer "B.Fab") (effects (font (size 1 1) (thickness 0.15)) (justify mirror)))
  (pad "1" smd roundrect (at -1.4625 0 90) (size 1.125 1.75) (layers "B.Cu" "B.Mask" "B.Paste") (roundrect_rratio 0.222222) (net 5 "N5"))
  (pad "2" smd roundrect (at 1.4625 0 90) (size 1.125 1.75) (layers "B.Cu" "B.Mask" "B.Paste") (roundrect_rratio 0.222222) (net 2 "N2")))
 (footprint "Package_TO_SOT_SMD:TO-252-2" (layer "B.Cu") (at 129.025 109.585 90)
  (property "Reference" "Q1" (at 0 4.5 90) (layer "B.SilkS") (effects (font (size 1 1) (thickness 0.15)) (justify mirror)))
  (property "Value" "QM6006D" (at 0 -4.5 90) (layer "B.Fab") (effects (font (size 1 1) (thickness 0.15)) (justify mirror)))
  (pad "" smd roundrect (at -0.415 -1.525 90) (size 3.05 2.75) (layers "B.Paste") (roundrect_rratio 0.090909))
  (pad "" smd roundrect (at -0.415 1.525 90) (size 3.05 2.75) (layers "B.Paste") (roundrect_rratio 0.090909))
  (pad "" smd roundrect (at 2.935 -1.525 90) (size 3.05 2.75) (layers "B.Paste") (roundrect_rratio 0.090909))
  (pad "" smd roundrect (at 2.935 1.525 90) (size 3.05 2.75) (layers "B.Paste") (roundrect_rratio 0.090909))
  (pad "1" smd roundrect (at -5.04 2.28 90) (size 2.2 1.2) (layers "B.Cu" "B.Mask" "B.Paste") (roundrect_rratio 0.208333) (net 8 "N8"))
  (pad "2" smd roundrect (at 1.26 0 90) (size 6.4 5.8) (layers "B.Cu" "B.Mask") (roundrect_rratio 0.043103) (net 11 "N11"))
  (pad "3" smd roundrect (at -5.04 -2.28 90) (size 2.2 1.2) (layers "B.Cu" "B.Mask" "B.Paste") (roundrect_rratio 0.208333) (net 7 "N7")))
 (gr_rect (start 108 76.5) (end 133 116.5) (stroke (width 0.05) (type default)) (fill no) (layer "Edge.Cuts"))
 (segment (start 113.7135 101.824) (end 116.01016 101.824) (width 0.2) (layer "B.Cu") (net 12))
 (segment (start 116.01016 101.824) (end 116.326 102.13984) (width 0.2) (layer "B.Cu") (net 12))
 (segment (start 114.68616 105.5) (end 113.5 105.5) (width 0.2) (layer "B.Cu") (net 12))
 (segment (start 112.5375 103) (end 113.7135 101.824) (width 0.2) (layer "B.Cu") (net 12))
 (segment (start 116.326 103.86016) (end 114.68616 105.5) (width 0.2) (layer "B.Cu") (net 12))
 (segment (start 116.326 102.13984) (end 116.326 103.86016) (width 0.2) (layer "B.Cu") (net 12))
 (segment (start 129.025 108.325) (end 113.675 108.325) (width 0.2) (layer "B.Cu") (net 11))
 (segment (start 113.675 108.325) (end 113.5 108.5) (width 0.2) (layer "B.Cu") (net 11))
 (segment (start 121.475 85.175) (end 116.325 85.175) (width 0.2) (layer "B.Cu") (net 3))
 (segment (start 116.325 85.175) (end 113.5 88) (width 0.2) (layer "B.Cu") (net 3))
 (segment (start 113.5 85) (end 115.5 87) (width 0.2) (layer "F.Cu") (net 4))
 (segment (start 115.5 87) (end 115.5 90) (width 0.2) (layer "F.Cu") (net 4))
 (segment (start 128 94.5) (end 129.176 95.676) (width 0.2) (layer "F.Cu") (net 2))
 (segment (start 129.176 97.91016) (end 128.08616 99) (width 0.2) (layer "F.Cu") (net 2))
 (segment (start 129.176 95.676) (end 129.176 97.91016) (width 0.2) (layer "F.Cu") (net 2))
 (segment (start 128.08616 99) (end 128 99) (width 0.2) (layer "F.Cu") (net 2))
 (segment (start 128.975 96.025) (end 128 97) (width 0.2) (layer "B.Cu") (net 1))
 (segment (start 128.975 85.1) (end 128.975 96.025) (width 0.2) (layer "B.Cu") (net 1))
 (segment (start 130.21676 93.574) (end 132.151 95.50824) (width 0.2) (layer "F.Cu") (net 7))
 (segment (start 132.151 109.349) (end 127 114.5) (width 0.2) (layer "F.Cu") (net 7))
 (segment (start 127.13984 93.574) (end 130.21676 93.574) (width 0.2) (layer "F.Cu") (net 7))
 (segment (start 125.12 95.59384) (end 127.13984 93.574) (width 0.2) (layer "F.Cu") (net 7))
 (segment (start 132.151 95.50824) (end 132.151 109.349) (width 0.2) (layer "F.Cu") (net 7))
 (segment (start 125.12 100.305) (end 125.12 92.685) (width 0.2) (layer "F.Cu") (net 7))
 (segment (start 122.58 92.685) (end 122.58 79.92) (width 0.2) (layer "F.Cu") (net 7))
 (segment (start 112.42 92.685) (end 114.96 92.685) (width 0.2) (layer "F.Cu") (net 7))
 (segment (start 125.12 100.305) (end 125.12 95.59384) (width 0.2) (layer "F.Cu") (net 7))
 (segment (start 110 89.055) (end 110 90.265) (width 0.2) (layer "F.Cu") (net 7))
 (segment (start 122.58 79.92) (end 123.5 79) (width 0.2) (layer "F.Cu") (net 7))
 (segment (start 120.04 92.685) (end 117.5 92.685) (width 0.2) (layer "F.Cu") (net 7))
 (segment (start 122.58 92.685) (end 120.04 92.685) (width 0.2) (layer "F.Cu") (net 7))
 (segment (start 110 90.265) (end 112.42 92.685) (width 0.2) (layer "F.Cu") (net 7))
 (segment (start 122.58 92.685) (end 125.12 92.685) (width 0.2) (layer "F.Cu") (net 7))
 (segment (start 125.88 93.445) (end 125.12 92.685) (width 0.2) (layer "F.Cu") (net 7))
 (segment (start 131 93.445) (end 125.88 93.445) (width 0.2) (layer "F.Cu") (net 7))
 (segment (start 114.96 92.685) (end 117.5 92.685) (width 0.2) (layer "F.Cu") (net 7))
 (segment (start 125.231 77.399) (end 123.755 78.875) (width 0.2) (layer "B.Cu") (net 7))
 (segment (start 126.745 114.625) (end 121.7 109.58) (width 0.2) (layer "B.Cu") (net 7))
 (segment (start 131.255 78.8) (end 129.854 77.399) (width 0.2) (layer "B.Cu") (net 7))
 (segment (start 129.854 77.399) (end 125.231 77.399) (width 0.2) (layer "B.Cu") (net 7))
 (segment (start 121.7 109.58) (end 110 109.58) (width 0.2) (layer "B.Cu") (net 7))
 (segment (start 113.859 96.664) (end 109.88 92.685) (width 0.2) (layer "F.Cu") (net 5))
 (segment (start 131 99) (end 127.5 102.5) (width 0.2) (layer "F.Cu") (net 5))
 (segment (start 127.5 102.5) (end 115.5 102.5) (width 0.2) (layer "F.Cu") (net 5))
 (segment (start 131 98.525) (end 131 99) (width 0.2) (layer "F.Cu") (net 5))
 (segment (start 115.5 102.5) (end 113.859 100.859) (width 0.2) (layer "F.Cu") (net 5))
 (segment (start 113.859 100.859) (end 113.859 96.664) (width 0.2) (layer "F.Cu") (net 5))
 (segment (start 115.4625 102.5375) (end 113.099 104.901) (width 0.2) (layer "B.Cu") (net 5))
 (segment (start 113.099 104.901) (end 113.099 105.6661) (width 0.2) (layer "B.Cu") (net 5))
 (segment (start 113.9625 104.5) (end 110 104.5) (width 0.2) (layer "B.Cu") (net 5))
 (segment (start 112.5375 90) (end 109.88 92.6575) (width 0.2) (layer "B.Cu") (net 5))
 (segment (start 113.3339 105.901) (end 124.024 105.901) (width 0.2) (layer "B.Cu") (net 5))
 (segment (start 124.024 105.901) (end 128 101.925) (width 0.2) (layer "B.Cu") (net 5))
 (segment (start 112.5375 90) (end 112.5375 86.5125) (width 0.2) (layer "B.Cu") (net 5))
 (segment (start 113.099 105.6661) (end 113.3339 105.901) (width 0.2) (layer "B.Cu") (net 5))
 (segment (start 115.4625 103) (end 115.4625 102.5375) (width 0.2) (layer "B.Cu") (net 5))
 (segment (start 109.88 92.6575) (end 109.88 92.685) (width 0.2) (layer "B.Cu") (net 5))
 (segment (start 112.5375 86.5125) (end 110 83.975) (width 0.2) (layer "B.Cu") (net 5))
 (segment (start 115.4625 103) (end 113.9625 104.5) (width 0.2) (layer "B.Cu") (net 5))
 (segment (start 108.779 87.736) (end 108.779 96.664) (width 0.2) (layer "F.Cu") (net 6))
 (segment (start 108.779 96.664) (end 112.42 100.305) (width 0.2) (layer "F.Cu") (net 6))
 (segment (start 110 86.515) (end 108.779 87.736) (width 0.2) (layer "F.Cu") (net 6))
 (segment (start 108.601 85.116) (end 110 86.515) (width 0.2) (layer "B.Cu") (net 6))
 (segment (start 119.195 78.875) (end 112.798 78.875) (width 0.2) (layer "B.Cu") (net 6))
 (segment (start 112.798 78.875) (end 108.601 83.072) (width 0.2) (layer "B.Cu") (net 6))
 (segment (start 108.601 83.072) (end 108.601 85.116) (width 0.2) (layer "B.Cu") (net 6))
 (segment (start 109.88 100.305) (end 108.849 101.336) (width 0.2) (layer "F.Cu") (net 8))
 (segment (start 108.849 101.336) (end 108.849 105.889) (width 0.2) (layer "F.Cu") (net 8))
 (segment (start 108.849 105.889) (end 110 107.04) (width 0.2) (layer "F.Cu") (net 8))
 (segment (start 131.305 114.625) (end 129.904 113.224) (width 0.2) (layer "B.Cu") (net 8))
 (segment (start 111.93612 108.97612) (end 110 107.04) (width 0.2) (layer "B.Cu") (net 8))
 (segment (start 129.904 113.224) (end 126.15984 113.224) (width 0.2) (layer "B.Cu") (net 8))
 (segment (start 126.15984 113.224) (end 121.91196 108.97612) (width 0.2) (layer "B.Cu") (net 8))
 (segment (start 121.91196 108.97612) (end 111.93612 108.97612) (width 0.2) (layer "B.Cu") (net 8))
 (segment (start 126.24726 101.406) (end 118.601 101.406) (width 0.2) (layer "F.Cu") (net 10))
 (segment (start 129.577 98.07626) (end 126.24726 101.406) (width 0.2) (layer "F.Cu") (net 10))
 (segment (start 129.577 97.408) (end 129.577 98.07626) (width 0.2) (layer "F.Cu") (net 10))
 (segment (start 118.601 101.406) (end 117.5 100.305) (width 0.2) (layer "F.Cu") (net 10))
 (segment (start 131 95.985) (end 129.577 97.408) (width 0.2) (layer "F.Cu") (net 10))
 (segment (start 132.176 94.809) (end 131 95.985) (width 0.2) (layer "B.Cu") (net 10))
 (segment (start 132.176 81.91484) (end 132.176 94.809) (width 0.2) (layer "B.Cu") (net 10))
 (segment (start 126.695 78.8) (end 129.06116 78.8) (width 0.2) (layer "B.Cu") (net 10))
 (segment (start 129.06116 78.8) (end 132.176 81.91484) (width 0.2) (layer "B.Cu") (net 10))
 (segment (start 116.061 99.204) (end 114.96 100.305) (width 0.2) (layer "F.Cu") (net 9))
 (segment (start 122.58 100.305) (end 121.479 99.204) (width 0.2) (layer "F.Cu") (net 9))
 (segment (start 120.04 100.305) (end 122.58 100.305) (width 0.2) (layer "F.Cu") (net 9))
 (segment (start 121.479 99.204) (end 116.061 99.204) (width 0.2) (layer "F.Cu") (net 9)))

